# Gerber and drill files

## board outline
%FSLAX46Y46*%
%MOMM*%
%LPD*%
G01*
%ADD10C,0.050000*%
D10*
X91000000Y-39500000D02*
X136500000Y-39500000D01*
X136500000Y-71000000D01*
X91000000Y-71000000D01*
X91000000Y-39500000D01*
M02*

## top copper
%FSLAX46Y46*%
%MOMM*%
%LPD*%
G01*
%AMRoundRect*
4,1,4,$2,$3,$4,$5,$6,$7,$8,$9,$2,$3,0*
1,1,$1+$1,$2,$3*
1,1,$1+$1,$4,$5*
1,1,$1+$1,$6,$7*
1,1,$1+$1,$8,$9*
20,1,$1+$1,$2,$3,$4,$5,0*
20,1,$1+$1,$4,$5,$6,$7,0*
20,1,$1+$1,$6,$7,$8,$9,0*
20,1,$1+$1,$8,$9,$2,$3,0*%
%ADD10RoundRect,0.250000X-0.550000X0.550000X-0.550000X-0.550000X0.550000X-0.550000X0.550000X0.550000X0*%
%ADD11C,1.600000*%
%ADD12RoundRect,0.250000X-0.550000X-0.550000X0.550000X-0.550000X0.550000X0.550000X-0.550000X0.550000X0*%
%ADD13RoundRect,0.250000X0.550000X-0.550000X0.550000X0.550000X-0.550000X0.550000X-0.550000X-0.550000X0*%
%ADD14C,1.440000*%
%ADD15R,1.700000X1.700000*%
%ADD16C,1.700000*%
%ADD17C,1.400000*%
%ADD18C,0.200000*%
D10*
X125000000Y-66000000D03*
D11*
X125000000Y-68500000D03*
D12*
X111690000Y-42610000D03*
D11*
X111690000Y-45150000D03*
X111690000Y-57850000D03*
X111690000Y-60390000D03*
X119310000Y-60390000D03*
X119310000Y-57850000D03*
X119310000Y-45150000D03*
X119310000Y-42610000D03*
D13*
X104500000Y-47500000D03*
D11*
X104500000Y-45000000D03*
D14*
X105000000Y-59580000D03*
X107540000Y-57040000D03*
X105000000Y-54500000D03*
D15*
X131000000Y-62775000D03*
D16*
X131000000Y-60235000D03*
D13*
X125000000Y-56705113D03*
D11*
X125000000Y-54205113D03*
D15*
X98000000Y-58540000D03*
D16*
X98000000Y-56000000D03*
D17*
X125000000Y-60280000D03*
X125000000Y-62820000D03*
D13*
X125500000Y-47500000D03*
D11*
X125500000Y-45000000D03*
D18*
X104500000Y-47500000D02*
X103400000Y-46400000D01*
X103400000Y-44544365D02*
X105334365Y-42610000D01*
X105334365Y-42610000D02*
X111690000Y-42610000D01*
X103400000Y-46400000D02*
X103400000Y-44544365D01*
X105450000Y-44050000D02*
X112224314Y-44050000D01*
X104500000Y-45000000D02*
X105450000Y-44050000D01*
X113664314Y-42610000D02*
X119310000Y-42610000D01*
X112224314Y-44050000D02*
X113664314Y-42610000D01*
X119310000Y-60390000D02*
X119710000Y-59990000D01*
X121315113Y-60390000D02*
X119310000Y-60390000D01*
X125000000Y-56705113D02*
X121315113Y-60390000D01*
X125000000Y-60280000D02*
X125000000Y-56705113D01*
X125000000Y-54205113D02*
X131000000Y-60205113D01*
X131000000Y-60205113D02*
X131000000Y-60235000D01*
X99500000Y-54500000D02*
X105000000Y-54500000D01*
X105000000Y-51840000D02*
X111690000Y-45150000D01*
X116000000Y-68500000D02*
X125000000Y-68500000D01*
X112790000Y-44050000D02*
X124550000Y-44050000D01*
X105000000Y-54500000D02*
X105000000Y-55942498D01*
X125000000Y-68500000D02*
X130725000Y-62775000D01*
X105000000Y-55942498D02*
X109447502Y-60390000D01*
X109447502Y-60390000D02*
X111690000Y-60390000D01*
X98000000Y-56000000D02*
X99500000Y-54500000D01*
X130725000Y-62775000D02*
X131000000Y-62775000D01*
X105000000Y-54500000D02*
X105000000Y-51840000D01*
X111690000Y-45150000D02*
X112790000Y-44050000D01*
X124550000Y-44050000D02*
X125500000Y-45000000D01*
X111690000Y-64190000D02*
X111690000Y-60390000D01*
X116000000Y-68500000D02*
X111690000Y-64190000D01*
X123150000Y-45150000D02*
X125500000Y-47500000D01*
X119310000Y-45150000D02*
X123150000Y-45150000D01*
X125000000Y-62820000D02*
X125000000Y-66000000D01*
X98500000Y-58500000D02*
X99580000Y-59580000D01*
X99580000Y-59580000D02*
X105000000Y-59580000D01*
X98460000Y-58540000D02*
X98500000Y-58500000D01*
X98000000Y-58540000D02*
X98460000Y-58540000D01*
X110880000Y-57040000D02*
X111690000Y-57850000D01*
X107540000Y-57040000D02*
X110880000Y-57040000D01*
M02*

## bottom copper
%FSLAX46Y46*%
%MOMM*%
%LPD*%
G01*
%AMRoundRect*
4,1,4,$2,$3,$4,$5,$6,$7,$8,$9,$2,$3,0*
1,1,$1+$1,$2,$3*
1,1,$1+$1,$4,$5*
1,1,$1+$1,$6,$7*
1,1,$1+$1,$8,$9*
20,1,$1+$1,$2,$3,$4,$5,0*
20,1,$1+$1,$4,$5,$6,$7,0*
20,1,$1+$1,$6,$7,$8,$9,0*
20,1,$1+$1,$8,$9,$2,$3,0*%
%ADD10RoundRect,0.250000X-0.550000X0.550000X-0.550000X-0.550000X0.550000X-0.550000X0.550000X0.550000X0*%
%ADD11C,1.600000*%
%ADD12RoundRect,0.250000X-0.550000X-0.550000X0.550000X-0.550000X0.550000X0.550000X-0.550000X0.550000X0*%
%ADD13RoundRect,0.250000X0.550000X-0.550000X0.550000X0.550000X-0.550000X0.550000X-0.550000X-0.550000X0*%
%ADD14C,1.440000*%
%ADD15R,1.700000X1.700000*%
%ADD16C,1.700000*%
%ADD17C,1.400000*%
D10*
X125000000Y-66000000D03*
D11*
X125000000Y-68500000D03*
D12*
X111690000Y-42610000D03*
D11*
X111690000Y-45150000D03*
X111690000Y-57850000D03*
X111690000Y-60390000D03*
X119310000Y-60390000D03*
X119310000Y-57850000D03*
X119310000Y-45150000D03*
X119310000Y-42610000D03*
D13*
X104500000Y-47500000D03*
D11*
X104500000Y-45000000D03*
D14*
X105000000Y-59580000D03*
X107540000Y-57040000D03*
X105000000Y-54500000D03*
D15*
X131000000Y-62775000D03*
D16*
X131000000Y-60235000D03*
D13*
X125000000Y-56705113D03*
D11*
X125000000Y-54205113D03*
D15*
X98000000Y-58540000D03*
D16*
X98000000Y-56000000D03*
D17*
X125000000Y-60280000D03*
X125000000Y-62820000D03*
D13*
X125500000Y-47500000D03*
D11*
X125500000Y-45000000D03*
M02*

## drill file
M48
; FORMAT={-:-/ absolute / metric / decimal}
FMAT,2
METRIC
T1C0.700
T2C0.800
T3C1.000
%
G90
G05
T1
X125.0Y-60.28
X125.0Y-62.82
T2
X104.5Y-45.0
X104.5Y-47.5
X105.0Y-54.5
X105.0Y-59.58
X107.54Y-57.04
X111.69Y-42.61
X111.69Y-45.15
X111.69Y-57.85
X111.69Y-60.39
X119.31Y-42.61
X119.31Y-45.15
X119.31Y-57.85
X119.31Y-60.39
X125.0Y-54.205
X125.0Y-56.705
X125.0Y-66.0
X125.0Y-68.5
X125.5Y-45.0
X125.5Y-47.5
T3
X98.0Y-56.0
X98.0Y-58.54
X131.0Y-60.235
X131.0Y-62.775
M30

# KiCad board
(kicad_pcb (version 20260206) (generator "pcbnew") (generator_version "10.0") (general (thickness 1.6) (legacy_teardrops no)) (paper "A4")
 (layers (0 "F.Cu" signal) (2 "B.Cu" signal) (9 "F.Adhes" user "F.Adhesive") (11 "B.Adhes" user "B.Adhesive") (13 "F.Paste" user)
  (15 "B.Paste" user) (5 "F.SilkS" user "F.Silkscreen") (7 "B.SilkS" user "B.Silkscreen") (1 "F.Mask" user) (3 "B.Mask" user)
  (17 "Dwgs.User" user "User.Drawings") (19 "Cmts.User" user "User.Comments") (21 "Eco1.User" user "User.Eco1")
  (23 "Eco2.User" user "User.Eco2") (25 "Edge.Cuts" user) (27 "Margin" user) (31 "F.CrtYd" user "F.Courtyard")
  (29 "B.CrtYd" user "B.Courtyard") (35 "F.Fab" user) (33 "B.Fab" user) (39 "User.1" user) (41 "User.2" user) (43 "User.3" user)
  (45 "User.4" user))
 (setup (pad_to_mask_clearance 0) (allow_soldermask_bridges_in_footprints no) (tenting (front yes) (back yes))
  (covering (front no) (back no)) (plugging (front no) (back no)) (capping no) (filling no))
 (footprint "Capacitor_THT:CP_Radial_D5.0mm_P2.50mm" (layer "F.Cu") (at 125 66 -90)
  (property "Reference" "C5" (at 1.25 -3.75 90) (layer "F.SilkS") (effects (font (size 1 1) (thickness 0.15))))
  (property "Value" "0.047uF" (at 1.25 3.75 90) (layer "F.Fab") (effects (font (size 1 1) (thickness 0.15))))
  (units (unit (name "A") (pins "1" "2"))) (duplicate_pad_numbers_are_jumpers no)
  (pad "1" thru_hole roundrect (at 0 0 270) (size 1.6 1.6) (drill 0.8) (layers "*.Cu" "*.Mask") (remove_unused_layers no)
   (roundrect_rratio 0.15625) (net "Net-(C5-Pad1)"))
  (pad "2" thru_hole circle (at 2.5 0 270) (size 1.6 1.6) (drill 0.8) (layers "*.Cu" "*.Mask") (remove_unused_layers no) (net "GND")))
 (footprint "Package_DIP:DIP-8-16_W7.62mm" (layer "F.Cu") (at 111.69 42.61)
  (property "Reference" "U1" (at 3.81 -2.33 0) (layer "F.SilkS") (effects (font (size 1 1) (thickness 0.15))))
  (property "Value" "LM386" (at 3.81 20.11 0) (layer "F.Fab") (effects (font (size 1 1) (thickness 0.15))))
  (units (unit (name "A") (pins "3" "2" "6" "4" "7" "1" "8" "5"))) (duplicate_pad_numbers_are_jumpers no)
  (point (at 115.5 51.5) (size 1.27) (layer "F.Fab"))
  (pad "1" thru_hole roundrect (at 0 0) (size 1.6 1.6) (drill 0.8) (layers "*.Cu" "*.Mask") (remove_unused_layers no)
   (roundrect_rratio 0.15625) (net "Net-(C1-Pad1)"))
  (pad "2" thru_hole circle (at 0 2.54) (size 1.6 1.6) (drill 0.8) (layers "*.Cu" "*.Mask") (remove_unused_layers no) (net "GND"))
  (pad "3" thru_hole circle (at 0 15.24) (size 1.6 1.6) (drill 0.8) (layers "*.Cu" "*.Mask") (remove_unused_layers no) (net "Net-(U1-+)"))
  (pad "4" thru_hole circle (at 0 17.78) (size 1.6 1.6) (drill 0.8) (layers "*.Cu" "*.Mask") (remove_unused_layers no) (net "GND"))
  (pad "5" thru_hole circle (at 7.62 17.78) (size 1.6 1.6) (drill 0.8) (layers "*.Cu" "*.Mask") (remove_unused_layers no)
   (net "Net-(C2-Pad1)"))
  (pad "6" thru_hole circle (at 7.62 15.24) (size 1.6 1.6) (drill 0.8) (layers "*.Cu" "*.Mask") (remove_unused_layers no) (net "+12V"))
  (pad "7" thru_hole circle (at 7.62 2.54) (size 1.6 1.6) (drill 0.8) (layers "*.Cu" "*.Mask") (remove_unused_layers no)
   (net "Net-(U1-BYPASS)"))
  (pad "8" thru_hole circle (at 7.62 0) (size 1.6 1.6) (drill 0.8) (layers "*.Cu" "*.Mask") (remove_unused_layers no) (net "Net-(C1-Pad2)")))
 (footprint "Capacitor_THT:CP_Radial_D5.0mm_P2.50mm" (layer "F.Cu") (at 104.5 47.5 90)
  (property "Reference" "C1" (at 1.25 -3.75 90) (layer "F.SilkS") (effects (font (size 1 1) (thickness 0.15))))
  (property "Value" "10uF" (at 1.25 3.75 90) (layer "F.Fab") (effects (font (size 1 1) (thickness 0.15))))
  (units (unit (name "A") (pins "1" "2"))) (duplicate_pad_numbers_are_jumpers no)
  (pad "1" thru_hole roundrect (at 0 0 90) (size 1.6 1.6) (drill 0.8) (layers "*.Cu" "*.Mask") (remove_unused_layers no)
   (roundrect_rratio 0.15625) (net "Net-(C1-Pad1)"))
  (pad "2" thru_hole circle (at 2.5 0 90) (size 1.6 1.6) (drill 0.8) (layers "*.Cu" "*.Mask") (remove_unused_layers no)
   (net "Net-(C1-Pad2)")))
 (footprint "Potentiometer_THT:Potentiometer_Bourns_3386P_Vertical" (layer "F.Cu") (at 105 59.58)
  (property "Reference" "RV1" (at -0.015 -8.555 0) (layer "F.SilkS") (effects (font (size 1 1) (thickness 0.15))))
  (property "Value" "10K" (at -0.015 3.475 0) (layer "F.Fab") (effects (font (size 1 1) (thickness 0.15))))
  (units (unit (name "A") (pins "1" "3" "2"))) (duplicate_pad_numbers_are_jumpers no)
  (pad "1" thru_hole circle (at 0 0) (size 1.44 1.44) (drill 0.8) (layers "*.Cu" "*.Mask") (remove_unused_layers no) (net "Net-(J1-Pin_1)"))
  (pad "2" thru_hole circle (at 2.54 -2.54) (size 1.44 1.44) (drill 0.8) (layers "*.Cu" "*.Mask") (remove_unused_layers no)
   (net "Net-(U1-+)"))
  (pad "3" thru_hole circle (at 0 -5.08) (size 1.44 1.44) (drill 0.8) (layers "*.Cu" "*.Mask") (remove_unused_layers no) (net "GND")))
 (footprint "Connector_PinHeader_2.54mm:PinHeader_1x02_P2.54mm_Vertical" (layer "F.Cu") (at 131 62.775 180)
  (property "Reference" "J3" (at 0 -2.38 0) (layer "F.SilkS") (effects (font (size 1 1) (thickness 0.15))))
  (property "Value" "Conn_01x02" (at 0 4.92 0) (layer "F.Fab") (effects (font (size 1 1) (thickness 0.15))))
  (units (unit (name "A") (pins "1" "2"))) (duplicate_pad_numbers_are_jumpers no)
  (pad "1" thru_hole rect (at 0 0 180) (size 1.7 1.7) (drill 1) (layers "*.Cu" "*.Mask") (remove_unused_layers no) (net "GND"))
  (pad "2" thru_hole circle (at 0 2.54 180) (size 1.7 1.7) (drill 1) (layers "*.Cu" "*.Mask") (remove_unused_layers no)
   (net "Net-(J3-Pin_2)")))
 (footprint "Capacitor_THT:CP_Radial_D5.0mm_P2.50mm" (layer "F.Cu") (at 125 56.705113 90)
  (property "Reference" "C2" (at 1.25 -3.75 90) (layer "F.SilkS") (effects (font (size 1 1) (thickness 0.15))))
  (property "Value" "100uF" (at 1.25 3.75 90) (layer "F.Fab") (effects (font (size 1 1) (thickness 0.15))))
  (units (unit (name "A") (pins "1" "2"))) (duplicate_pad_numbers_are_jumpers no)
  (pad "1" thru_hole roundrect (at 0 0 90) (size 1.6 1.6) (drill 0.8) (layers "*.Cu" "*.Mask") (remove_unused_layers no)
   (roundrect_rratio 0.15625) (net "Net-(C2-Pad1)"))
  (pad "2" thru_hole circle (at 2.5 0 90) (size 1.6 1.6) (drill 0.8) (layers "*.Cu" "*.Mask") (remove_unused_layers no)
   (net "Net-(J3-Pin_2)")))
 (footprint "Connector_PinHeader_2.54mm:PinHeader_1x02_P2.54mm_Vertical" (layer "F.Cu") (at 98 58.54 180)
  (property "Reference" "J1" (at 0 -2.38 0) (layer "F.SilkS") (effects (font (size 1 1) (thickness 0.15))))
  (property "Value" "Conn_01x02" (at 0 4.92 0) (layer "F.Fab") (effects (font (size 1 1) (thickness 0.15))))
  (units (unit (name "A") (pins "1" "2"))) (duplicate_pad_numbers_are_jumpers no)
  (pad "1" thru_hole rect (at 0 0 180) (size 1.7 1.7) (drill 1) (layers "*.Cu" "*.Mask") (remove_unused_layers no) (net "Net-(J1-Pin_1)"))
  (pad "2" thru_hole circle (at 0 2.54 180) (size 1.7 1.7) (drill 1) (layers "*.Cu" "*.Mask") (remove_unused_layers no) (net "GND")))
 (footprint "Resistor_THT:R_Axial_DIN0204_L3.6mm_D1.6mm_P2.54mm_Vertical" (layer "F.Cu") (at 125 60.28 -90)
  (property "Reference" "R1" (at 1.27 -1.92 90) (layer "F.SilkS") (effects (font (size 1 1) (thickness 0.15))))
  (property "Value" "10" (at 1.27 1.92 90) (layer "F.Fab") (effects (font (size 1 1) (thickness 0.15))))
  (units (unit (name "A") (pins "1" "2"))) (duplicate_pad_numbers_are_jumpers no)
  (pad "1" thru_hole circle (at 0 0 270) (size 1.4 1.4) (drill 0.7) (layers "*.Cu" "*.Mask") (remove_unused_layers no) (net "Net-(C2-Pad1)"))
  (pad "2" thru_hole circle (at 2.54 0 270) (size 1.4 1.4) (drill 0.7) (layers "*.Cu" "*.Mask") (remove_unused_layers no)
   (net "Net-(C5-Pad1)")))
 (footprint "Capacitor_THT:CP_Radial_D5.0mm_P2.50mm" (layer "F.Cu") (at 125.5 47.5 90)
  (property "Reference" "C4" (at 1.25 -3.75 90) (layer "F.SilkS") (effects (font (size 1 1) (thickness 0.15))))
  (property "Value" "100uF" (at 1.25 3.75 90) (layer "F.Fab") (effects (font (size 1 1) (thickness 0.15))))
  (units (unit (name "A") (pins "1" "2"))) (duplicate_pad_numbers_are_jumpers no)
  (pad "1" thru_hole roundrect (at 0 0 90) (size 1.6 1.6) (drill 0.8) (layers "*.Cu" "*.Mask") (remove_unused_layers no)
   (roundrect_rratio 0.15625) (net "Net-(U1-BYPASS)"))
  (pad "2" thru_hole circle (at 2.5 0 90) (size 1.6 1.6) (drill 0.8) (layers "*.Cu" "*.Mask") (remove_unused_layers no) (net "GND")))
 (gr_rect (start 91 39.5) (end 136.5 71) (stroke (width 0.05) (type default)) (fill no) (layer "Edge.Cuts"))
 (segment (start 104.5 47.5) (end 103.4 46.4) (width 0.2) (layer "F.Cu") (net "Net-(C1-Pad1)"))
 (segment (start 103.4 44.544365) (end 105.334365 42.61) (width 0.2) (layer "F.Cu") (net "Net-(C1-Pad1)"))
 (segment (start 105.334365 42.61) (end 111.69 42.61) (width 0.2) (layer "F.Cu") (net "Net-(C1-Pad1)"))
 (segment (start 103.4 46.4) (end 103.4 44.544365) (width 0.2) (layer "F.Cu") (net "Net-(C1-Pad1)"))
 (segment (start 105.45 44.05) (end 112.224314 44.05) (width 0.2) (layer "F.Cu") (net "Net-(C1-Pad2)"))
 (segment (start 104.5 45) (end 105.45 44.05) (width 0.2) (layer "F.Cu") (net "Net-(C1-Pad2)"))
 (segment (start 113.664314 42.61) (end 119.31 42.61) (width 0.2) (layer "F.Cu") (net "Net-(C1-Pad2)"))
 (segment (start 112.224314 44.05) (end 113.664314 42.61) (width 0.2) (layer "F.Cu") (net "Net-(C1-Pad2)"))
 (segment (start 119.31 60.39) (end 119.71 59.99) (width 0.2) (layer "F.Cu") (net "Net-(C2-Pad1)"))
 (segment (start 121.315113 60.39) (end 119.31 60.39) (width 0.2) (layer "F.Cu") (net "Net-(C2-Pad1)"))
 (segment (start 125 56.705113) (end 121.315113 60.39) (width 0.2) (layer "F.Cu") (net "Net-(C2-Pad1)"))
 (segment (start 125 60.28) (end 125 56.705113) (width 0.2) (layer "F.Cu") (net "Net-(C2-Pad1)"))
 (segment (start 125 54.205113) (end 131 60.205113) (width 0.2) (layer "F.Cu") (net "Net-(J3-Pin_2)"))
 (segment (start 131 60.205113) (end 131 60.235) (width 0.2) (layer "F.Cu") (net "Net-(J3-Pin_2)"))
 (segment (start 99.5 54.5) (end 105 54.5) (width 0.2) (layer "F.Cu") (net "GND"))
 (segment (start 105 51.84) (end 111.69 45.15) (width 0.2) (layer "F.Cu") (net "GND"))
 (segment (start 116 68.5) (end 125 68.5) (width 0.2) (layer "F.Cu") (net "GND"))
 (segment (start 112.79 44.05) (end 124.55 44.05) (width 0.2) (layer "F.Cu") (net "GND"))
 (segment (start 105 54.5) (end 105 55.942498) (width 0.2) (layer "F.Cu") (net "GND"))
 (segment (start 125 68.5) (end 130.725 62.775) (width 0.2) (layer "F.Cu") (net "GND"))
 (segment (start 105 55.942498) (end 109.447502 60.39) (width 0.2) (layer "F.Cu") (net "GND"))
 (segment (start 109.447502 60.39) (end 111.69 60.39) (width 0.2) (layer "F.Cu") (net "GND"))
 (segment (start 98 56) (end 99.5 54.5) (width 0.2) (layer "F.Cu") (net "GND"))
 (segment (start 130.725 62.775) (end 131 62.775) (width 0.2) (layer "F.Cu") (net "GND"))
 (segment (start 105 54.5) (end 105 51.84) (width 0.2) (layer "F.Cu") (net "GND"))
 (segment (start 111.69 45.15) (end 112.79 44.05) (width 0.2) (layer "F.Cu") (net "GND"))
 (segment (start 124.55 44.05) (end 125.5 45) (width 0.2) (layer "F.Cu") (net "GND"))
 (segment (start 111.69 64.19) (end 111.69 60.39) (width 0.2) (layer "F.Cu") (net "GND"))
 (segment (start 116 68.5) (end 111.69 64.19) (width 0.2) (layer "F.Cu") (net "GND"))
 (segment (start 123.15 45.15) (end 125.5 47.5) (width 0.2) (layer "F.Cu") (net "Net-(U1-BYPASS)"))
 (segment (start 119.31 45.15) (end 123.15 45.15) (width 0.2) (layer "F.Cu") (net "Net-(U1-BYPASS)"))
 (segment (start 125 62.82) (end 125 66) (width 0.2) (layer "F.Cu") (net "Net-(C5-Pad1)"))
 (segment (start 98.5 58.5) (end 99.58 59.58) (width 0.2) (layer "F.Cu") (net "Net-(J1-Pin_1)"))
 (segment (start 99.58 59.58) (end 105 59.58) (width 0.2) (layer "F.Cu") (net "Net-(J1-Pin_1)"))
 (segment (start 98.46 58.54) (end 98.5 58.5) (width 0.2) (layer "F.Cu") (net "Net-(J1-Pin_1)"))
 (segment (start 98 58.54) (end 98.46 58.54) (width 0.2) (layer "F.Cu") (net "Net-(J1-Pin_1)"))
 (segment (start 110.88 57.04) (end 111.69 57.85) (width 0.2) (layer "F.Cu") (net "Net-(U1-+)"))
 (segment (start 107.54 57.04) (end 110.88 57.04) (width 0.2) (layer "F.Cu") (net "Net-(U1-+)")))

